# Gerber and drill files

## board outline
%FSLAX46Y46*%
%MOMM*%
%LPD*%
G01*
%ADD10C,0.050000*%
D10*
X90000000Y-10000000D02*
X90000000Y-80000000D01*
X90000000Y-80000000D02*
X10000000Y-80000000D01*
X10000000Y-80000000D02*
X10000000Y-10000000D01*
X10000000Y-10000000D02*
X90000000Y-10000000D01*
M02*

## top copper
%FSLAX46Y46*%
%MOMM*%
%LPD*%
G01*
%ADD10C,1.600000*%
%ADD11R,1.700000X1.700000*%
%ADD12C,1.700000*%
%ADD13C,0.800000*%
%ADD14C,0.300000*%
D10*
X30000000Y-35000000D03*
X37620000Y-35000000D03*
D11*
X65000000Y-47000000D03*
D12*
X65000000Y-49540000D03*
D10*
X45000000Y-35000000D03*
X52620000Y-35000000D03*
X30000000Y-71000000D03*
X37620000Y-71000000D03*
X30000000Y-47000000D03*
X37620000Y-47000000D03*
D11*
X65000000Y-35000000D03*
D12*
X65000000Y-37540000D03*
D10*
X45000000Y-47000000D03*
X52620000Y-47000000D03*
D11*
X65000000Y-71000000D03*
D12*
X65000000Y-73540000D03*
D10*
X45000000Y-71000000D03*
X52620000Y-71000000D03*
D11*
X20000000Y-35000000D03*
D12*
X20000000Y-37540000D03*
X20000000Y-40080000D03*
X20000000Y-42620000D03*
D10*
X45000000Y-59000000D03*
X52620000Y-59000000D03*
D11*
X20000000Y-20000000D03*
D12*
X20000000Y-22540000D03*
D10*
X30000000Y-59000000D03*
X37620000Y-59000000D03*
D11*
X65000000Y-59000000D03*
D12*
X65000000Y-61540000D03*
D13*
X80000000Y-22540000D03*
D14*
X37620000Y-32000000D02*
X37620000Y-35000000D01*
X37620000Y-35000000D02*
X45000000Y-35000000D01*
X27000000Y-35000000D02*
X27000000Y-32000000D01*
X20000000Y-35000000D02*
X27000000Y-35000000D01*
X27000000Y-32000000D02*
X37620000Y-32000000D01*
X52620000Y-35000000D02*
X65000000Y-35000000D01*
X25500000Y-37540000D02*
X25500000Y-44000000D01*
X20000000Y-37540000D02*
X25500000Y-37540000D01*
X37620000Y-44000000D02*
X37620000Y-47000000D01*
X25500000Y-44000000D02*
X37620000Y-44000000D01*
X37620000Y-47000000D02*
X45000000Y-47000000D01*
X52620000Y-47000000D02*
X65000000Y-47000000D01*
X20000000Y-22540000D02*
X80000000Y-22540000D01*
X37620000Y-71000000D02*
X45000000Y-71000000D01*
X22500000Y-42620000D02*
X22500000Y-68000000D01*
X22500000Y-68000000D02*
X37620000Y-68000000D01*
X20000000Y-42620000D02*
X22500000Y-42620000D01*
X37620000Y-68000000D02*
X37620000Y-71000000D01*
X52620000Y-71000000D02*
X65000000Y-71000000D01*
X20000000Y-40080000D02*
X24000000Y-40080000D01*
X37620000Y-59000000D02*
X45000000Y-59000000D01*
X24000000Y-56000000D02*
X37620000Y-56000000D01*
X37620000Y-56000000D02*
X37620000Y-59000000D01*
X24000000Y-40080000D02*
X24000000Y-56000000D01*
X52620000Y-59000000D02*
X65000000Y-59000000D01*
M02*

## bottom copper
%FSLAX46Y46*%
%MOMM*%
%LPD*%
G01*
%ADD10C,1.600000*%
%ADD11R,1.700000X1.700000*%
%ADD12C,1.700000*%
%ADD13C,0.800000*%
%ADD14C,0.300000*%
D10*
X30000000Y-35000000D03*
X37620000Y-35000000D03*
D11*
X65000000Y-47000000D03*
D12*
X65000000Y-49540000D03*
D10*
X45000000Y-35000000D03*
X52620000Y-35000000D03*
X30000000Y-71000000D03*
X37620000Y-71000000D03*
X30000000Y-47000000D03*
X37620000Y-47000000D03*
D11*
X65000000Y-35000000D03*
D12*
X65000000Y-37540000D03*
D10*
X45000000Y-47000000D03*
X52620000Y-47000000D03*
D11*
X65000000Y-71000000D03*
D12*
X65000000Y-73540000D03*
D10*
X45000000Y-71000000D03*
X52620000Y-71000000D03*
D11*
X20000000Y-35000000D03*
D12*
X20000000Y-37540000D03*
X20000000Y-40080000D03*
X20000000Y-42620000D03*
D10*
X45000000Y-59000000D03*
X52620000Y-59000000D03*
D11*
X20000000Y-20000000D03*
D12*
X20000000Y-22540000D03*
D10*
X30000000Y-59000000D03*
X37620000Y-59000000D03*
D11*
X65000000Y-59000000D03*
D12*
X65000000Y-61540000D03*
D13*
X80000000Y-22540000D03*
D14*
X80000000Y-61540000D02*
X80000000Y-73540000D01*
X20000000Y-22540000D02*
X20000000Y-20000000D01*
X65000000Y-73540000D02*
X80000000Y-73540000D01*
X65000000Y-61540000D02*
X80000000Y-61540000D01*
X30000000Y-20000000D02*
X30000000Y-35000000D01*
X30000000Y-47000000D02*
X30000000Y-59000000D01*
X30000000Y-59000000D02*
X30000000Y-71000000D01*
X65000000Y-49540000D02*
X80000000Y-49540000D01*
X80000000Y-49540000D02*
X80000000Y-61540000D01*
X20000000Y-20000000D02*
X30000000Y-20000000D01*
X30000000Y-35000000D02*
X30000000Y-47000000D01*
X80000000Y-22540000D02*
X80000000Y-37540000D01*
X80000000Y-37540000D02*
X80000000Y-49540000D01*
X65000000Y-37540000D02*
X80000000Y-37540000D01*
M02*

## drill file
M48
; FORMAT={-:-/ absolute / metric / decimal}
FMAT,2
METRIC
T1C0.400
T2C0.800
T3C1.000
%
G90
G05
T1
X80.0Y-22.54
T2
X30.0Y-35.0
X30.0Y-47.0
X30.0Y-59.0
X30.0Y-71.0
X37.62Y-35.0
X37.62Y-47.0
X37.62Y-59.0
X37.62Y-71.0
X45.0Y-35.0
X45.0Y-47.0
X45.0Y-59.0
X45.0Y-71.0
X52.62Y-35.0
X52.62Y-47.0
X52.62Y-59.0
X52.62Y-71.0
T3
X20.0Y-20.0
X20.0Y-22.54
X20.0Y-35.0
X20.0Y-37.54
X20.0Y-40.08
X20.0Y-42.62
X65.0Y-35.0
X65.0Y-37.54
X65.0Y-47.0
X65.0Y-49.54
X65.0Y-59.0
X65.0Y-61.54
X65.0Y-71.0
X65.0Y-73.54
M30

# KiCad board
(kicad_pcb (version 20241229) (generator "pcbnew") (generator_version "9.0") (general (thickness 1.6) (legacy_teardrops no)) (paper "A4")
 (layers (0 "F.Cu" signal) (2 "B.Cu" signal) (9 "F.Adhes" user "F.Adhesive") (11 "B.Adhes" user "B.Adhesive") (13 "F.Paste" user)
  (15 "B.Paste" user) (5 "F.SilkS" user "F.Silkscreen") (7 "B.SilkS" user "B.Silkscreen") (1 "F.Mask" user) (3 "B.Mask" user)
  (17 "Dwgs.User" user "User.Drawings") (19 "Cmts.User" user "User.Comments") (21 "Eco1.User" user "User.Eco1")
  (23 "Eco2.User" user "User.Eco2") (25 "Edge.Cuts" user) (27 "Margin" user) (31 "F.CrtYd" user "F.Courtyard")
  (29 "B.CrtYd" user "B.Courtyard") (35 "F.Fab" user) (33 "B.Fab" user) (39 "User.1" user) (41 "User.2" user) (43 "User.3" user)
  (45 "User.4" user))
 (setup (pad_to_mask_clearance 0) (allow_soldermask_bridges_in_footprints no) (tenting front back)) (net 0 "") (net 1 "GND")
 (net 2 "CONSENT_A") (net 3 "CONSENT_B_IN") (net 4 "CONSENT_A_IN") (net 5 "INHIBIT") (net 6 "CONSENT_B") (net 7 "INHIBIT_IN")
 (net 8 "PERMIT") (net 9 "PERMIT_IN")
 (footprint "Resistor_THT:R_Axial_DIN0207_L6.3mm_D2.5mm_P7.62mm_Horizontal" (layer "F.Cu") (at 30 35)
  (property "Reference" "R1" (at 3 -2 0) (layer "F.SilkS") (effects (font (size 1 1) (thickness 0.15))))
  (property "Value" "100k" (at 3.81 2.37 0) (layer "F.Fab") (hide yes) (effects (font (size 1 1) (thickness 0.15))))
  (pad "1" thru_hole circle (at 0 0) (size 1.6 1.6) (drill 0.8) (layers "*.Cu" "*.Mask") (remove_unused_layers no) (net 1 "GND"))
  (pad "2" thru_hole circle (at 7.62 0) (size 1.6 1.6) (drill 0.8) (layers "*.Cu" "*.Mask") (remove_unused_layers no) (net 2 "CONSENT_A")))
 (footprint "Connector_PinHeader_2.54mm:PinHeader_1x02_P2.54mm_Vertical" (layer "F.Cu") (at 65 47)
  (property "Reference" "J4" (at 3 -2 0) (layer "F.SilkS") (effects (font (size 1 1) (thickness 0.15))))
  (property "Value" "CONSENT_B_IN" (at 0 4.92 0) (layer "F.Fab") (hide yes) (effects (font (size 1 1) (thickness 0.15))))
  (pad "1" thru_hole rect (at 0 0) (size 1.7 1.7) (drill 1) (layers "*.Cu" "*.Mask") (remove_unused_layers no) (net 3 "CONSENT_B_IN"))
  (pad "2" thru_hole circle (at 0 2.54) (size 1.7 1.7) (drill 1) (layers "*.Cu" "*.Mask") (remove_unused_layers no) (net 1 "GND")))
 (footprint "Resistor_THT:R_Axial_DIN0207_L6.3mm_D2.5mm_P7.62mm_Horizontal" (layer "F.Cu") (at 45 35)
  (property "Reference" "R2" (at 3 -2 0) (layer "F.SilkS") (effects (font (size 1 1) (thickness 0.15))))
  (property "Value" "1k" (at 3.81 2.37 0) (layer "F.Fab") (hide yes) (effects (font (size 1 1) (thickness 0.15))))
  (pad "1" thru_hole circle (at 0 0) (size 1.6 1.6) (drill 0.8) (layers "*.Cu" "*.Mask") (remove_unused_layers no) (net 2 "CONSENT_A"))
  (pad "2" thru_hole circle (at 7.62 0) (size 1.6 1.6) (drill 0.8) (layers "*.Cu" "*.Mask") (remove_unused_layers no) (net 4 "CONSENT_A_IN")))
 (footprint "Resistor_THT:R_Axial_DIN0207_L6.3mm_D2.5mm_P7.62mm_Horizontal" (layer "F.Cu") (at 30 71)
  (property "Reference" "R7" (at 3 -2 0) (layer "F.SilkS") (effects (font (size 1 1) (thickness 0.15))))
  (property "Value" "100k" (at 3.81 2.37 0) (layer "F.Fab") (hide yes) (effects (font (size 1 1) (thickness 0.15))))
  (pad "1" thru_hole circle (at 0 0) (size 1.6 1.6) (drill 0.8) (layers "*.Cu" "*.Mask") (remove_unused_layers no) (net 1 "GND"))
  (pad "2" thru_hole circle (at 7.62 0) (size 1.6 1.6) (drill 0.8) (layers "*.Cu" "*.Mask") (remove_unused_layers no) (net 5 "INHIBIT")))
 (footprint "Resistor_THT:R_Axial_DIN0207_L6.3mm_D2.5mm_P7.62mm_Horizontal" (layer "F.Cu") (at 30 47)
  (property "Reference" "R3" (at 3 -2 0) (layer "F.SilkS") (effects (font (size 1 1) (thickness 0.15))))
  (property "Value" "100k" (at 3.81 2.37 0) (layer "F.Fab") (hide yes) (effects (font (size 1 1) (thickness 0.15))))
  (pad "1" thru_hole circle (at 0 0) (size 1.6 1.6) (drill 0.8) (layers "*.Cu" "*.Mask") (remove_unused_layers no) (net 1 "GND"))
  (pad "2" thru_hole circle (at 7.62 0) (size 1.6 1.6) (drill 0.8) (layers "*.Cu" "*.Mask") (remove_unused_layers no) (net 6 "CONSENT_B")))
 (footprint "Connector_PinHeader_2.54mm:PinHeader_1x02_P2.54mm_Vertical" (layer "F.Cu") (at 65 35)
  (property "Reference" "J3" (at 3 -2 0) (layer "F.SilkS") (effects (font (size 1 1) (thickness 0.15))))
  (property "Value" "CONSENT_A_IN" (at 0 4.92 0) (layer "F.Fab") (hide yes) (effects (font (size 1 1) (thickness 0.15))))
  (pad "1" thru_hole rect (at 0 0) (size 1.7 1.7) (drill 1) (layers "*.Cu" "*.Mask") (remove_unused_layers no) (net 4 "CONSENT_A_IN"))
  (pad "2" thru_hole circle (at 0 2.54) (size 1.7 1.7) (drill 1) (layers "*.Cu" "*.Mask") (remove_unused_layers no) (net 1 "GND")))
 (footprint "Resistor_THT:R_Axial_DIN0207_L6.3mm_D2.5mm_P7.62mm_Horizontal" (layer "F.Cu") (at 45 47)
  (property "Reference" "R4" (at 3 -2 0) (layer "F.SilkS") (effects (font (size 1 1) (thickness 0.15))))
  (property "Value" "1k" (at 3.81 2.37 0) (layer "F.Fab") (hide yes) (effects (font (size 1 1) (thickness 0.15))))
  (pad "1" thru_hole circle (at 0 0) (size 1.6 1.6) (drill 0.8) (layers "*.Cu" "*.Mask") (remove_unused_layers no) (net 6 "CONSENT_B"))
  (pad "2" thru_hole circle (at 7.62 0) (size 1.6 1.6) (drill 0.8) (layers "*.Cu" "*.Mask") (remove_unused_layers no) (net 3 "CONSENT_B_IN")))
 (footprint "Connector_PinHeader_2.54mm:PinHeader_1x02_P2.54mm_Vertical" (layer "F.Cu") (at 65 71)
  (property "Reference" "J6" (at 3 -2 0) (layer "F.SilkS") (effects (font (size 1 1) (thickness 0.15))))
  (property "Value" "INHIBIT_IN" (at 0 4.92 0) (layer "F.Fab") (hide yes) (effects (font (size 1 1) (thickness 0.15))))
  (pad "1" thru_hole rect (at 0 0) (size 1.7 1.7) (drill 1) (layers "*.Cu" "*.Mask") (remove_unused_layers no) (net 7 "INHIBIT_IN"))
  (pad "2" thru_hole circle (at 0 2.54) (size 1.7 1.7) (drill 1) (layers "*.Cu" "*.Mask") (remove_unused_layers no) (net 1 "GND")))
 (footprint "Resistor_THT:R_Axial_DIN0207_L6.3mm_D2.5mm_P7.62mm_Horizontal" (layer "F.Cu") (at 45 71)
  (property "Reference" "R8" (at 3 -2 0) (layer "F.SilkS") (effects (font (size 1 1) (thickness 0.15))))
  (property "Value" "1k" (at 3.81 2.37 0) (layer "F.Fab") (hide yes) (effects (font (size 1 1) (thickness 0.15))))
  (pad "1" thru_hole circle (at 0 0) (size 1.6 1.6) (drill 0.8) (layers "*.Cu" "*.Mask") (remove_unused_layers no) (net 5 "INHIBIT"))
  (pad "2" thru_hole circle (at 7.62 0) (size 1.6 1.6) (drill 0.8) (layers "*.Cu" "*.Mask") (remove_unused_layers no) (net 7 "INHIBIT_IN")))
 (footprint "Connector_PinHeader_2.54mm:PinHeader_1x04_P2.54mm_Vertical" (layer "F.Cu") (at 20 35)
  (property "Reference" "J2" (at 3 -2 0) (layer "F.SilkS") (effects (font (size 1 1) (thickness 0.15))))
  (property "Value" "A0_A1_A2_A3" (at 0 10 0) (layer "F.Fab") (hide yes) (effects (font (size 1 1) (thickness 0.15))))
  (pad "1" thru_hole rect (at 0 0) (size 1.7 1.7) (drill 1) (layers "*.Cu" "*.Mask") (remove_unused_layers no) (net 2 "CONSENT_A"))
  (pad "2" thru_hole circle (at 0 2.54) (size 1.7 1.7) (drill 1) (layers "*.Cu" "*.Mask") (remove_unused_layers no) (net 6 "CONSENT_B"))
  (pad "3" thru_hole circle (at 0 5.08) (size 1.7 1.7) (drill 1) (layers "*.Cu" "*.Mask") (remove_unused_layers no) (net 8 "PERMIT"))
  (pad "4" thru_hole circle (at 0 7.62) (size 1.7 1.7) (drill 1) (layers "*.Cu" "*.Mask") (remove_unused_layers no) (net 5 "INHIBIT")))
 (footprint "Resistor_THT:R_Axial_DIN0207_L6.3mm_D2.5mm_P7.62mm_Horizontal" (layer "F.Cu") (at 45 59)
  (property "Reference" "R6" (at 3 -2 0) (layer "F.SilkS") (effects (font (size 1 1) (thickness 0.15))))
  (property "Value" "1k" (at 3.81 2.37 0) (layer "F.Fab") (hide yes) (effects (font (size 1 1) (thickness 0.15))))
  (pad "1" thru_hole circle (at 0 0) (size 1.6 1.6) (drill 0.8) (layers "*.Cu" "*.Mask") (remove_unused_layers no) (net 8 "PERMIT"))
  (pad "2" thru_hole circle (at 7.62 0) (size 1.6 1.6) (drill 0.8) (layers "*.Cu" "*.Mask") (remove_unused_layers no) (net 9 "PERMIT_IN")))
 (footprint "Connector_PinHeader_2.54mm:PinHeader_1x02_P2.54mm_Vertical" (layer "F.Cu") (at 20 20)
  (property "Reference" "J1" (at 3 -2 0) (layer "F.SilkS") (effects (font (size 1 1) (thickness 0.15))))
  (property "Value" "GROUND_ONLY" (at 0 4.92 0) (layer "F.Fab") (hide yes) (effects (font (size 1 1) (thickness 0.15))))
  (pad "1" thru_hole rect (at 0 0) (size 1.7 1.7) (drill 1) (layers "*.Cu" "*.Mask") (remove_unused_layers no) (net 1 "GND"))
  (pad "2" thru_hole circle (at 0 2.54) (size 1.7 1.7) (drill 1) (layers "*.Cu" "*.Mask") (remove_unused_layers no) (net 1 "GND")))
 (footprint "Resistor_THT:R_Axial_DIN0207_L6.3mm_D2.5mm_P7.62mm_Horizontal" (layer "F.Cu") (at 30 59)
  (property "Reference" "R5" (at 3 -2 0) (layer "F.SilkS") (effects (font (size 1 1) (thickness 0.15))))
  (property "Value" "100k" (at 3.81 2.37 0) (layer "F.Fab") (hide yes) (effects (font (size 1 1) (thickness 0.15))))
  (pad "1" thru_hole circle (at 0 0) (size 1.6 1.6) (drill 0.8) (layers "*.Cu" "*.Mask") (remove_unused_layers no) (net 1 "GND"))
  (pad "2" thru_hole circle (at 7.62 0) (size 1.6 1.6) (drill 0.8) (layers "*.Cu" "*.Mask") (remove_unused_layers no) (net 8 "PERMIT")))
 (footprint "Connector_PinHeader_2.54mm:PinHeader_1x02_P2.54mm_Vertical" (layer "F.Cu") (at 65 59)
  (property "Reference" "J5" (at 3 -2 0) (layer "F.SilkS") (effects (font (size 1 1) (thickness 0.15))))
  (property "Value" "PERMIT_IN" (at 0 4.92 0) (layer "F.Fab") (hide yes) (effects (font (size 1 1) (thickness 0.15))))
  (pad "1" thru_hole rect (at 0 0) (size 1.7 1.7) (drill 1) (layers "*.Cu" "*.Mask") (remove_unused_layers no) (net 9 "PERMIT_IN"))
  (pad "2" thru_hole circle (at 0 2.54) (size 1.7 1.7) (drill 1) (layers "*.Cu" "*.Mask") (remove_unused_layers no) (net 1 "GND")))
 (gr_line (start 90 10) (end 90 80) (stroke (width 0.05) (type default)) (layer "Edge.Cuts"))
 (gr_line (start 90 80) (end 10 80) (stroke (width 0.05) (type default)) (layer "Edge.Cuts"))
 (gr_line (start 10 80) (end 10 10) (stroke (width 0.05) (type default)) (layer "Edge.Cuts"))
 (gr_line (start 10 10) (end 90 10) (stroke (width 0.05) (type default)) (layer "Edge.Cuts"))
 (segment (start 37.62 32) (end 37.62 35) (width 0.3) (layer "F.Cu") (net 2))
 (segment (start 37.62 35) (end 45 35) (width 0.3) (layer "F.Cu") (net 2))
 (segment (start 27 35) (end 27 32) (width 0.3) (layer "F.Cu") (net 2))
 (segment (start 20 35) (end 27 35) (width 0.3) (layer "F.Cu") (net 2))
 (segment (start 27 32) (end 37.62 32) (width 0.3) (layer "F.Cu") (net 2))
 (segment (start 52.62 35) (end 65 35) (width 0.3) (layer "F.Cu") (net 4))
 (segment (start 25.5 37.54) (end 25.5 44) (width 0.3) (layer "F.Cu") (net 6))
 (segment (start 20 37.54) (end 25.5 37.54) (width 0.3) (layer "F.Cu") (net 6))
 (segment (start 37.62 44) (end 37.62 47) (width 0.3) (layer "F.Cu") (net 6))
 (segment (start 25.5 44) (end 37.62 44) (width 0.3) (layer "F.Cu") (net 6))
 (segment (start 37.62 47) (end 45 47) (width 0.3) (layer "F.Cu") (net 6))
 (segment (start 52.62 47) (end 65 47) (width 0.3) (layer "F.Cu") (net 3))
 (segment (start 20 22.54) (end 80 22.54) (width 0.3) (layer "F.Cu") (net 1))
 (via (at 80 22.54) (size 0.8) (drill 0.4) (layers "F.Cu" "B.Cu") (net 1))
 (segment (start 80 61.54) (end 80 73.54) (width 0.3) (layer "B.Cu") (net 1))
 (segment (start 20 22.54) (end 20 20) (width 0.3) (layer "B.Cu") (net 1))
 (segment (start 65 73.54) (end 80 73.54) (width 0.3) (layer "B.Cu") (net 1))
 (segment (start 65 61.54) (end 80 61.54) (width 0.3) (layer "B.Cu") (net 1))
 (segment (start 30 20) (end 30 35) (width 0.3) (layer "B.Cu") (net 1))
 (segment (start 30 47) (end 30 59) (width 0.3) (layer "B.Cu") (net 1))
 (segment (start 30 59) (end 30 71) (width 0.3) (layer "B.Cu") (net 1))
 (segment (start 65 49.54) (end 80 49.54) (width 0.3) (layer "B.Cu") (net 1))
 (segment (start 80 49.54) (end 80 61.54) (width 0.3) (layer "B.Cu") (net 1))
 (segment (start 20 20) (end 30 20) (width 0.3) (layer "B.Cu") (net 1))
 (segment (start 30 35) (end 30 47) (width 0.3) (layer "B.Cu") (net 1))
 (segment (start 80 22.54) (end 80 37.54) (width 0.3) (layer "B.Cu") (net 1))
 (segment (start 80 37.54) (end 80 49.54) (width 0.3) (layer "B.Cu") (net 1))
 (segment (start 65 37.54) (end 80 37.54) (width 0.3) (layer "B.Cu") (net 1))
 (segment (start 37.62 71) (end 45 71) (width 0.3) (layer "F.Cu") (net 5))
 (segment (start 22.5 42.62) (end 22.5 68) (width 0.3) (layer "F.Cu") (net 5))
 (segment (start 22.5 68) (end 37.62 68) (width 0.3) (layer "F.Cu") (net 5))
 (segment (start 20 42.62) (end 22.5 42.62) (width 0.3) (layer "F.Cu") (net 5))
 (segment (start 37.62 68) (end 37.62 71) (width 0.3) (layer "F.Cu") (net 5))
 (segment (start 52.62 71) (end 65 71) (width 0.3) (layer "F.Cu") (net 7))
 (segment (start 20 40.08) (end 24 40.08) (width 0.3) (layer "F.Cu") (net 8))
 (segment (start 37.62 59) (end 45 59) (width 0.3) (layer "F.Cu") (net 8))
 (segment (start 24 56) (end 37.62 56) (width 0.3) (layer "F.Cu") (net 8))
 (segment (start 37.62 56) (end 37.62 59) (width 0.3) (layer "F.Cu") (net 8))
 (segment (start 24 40.08) (end 24 56) (width 0.3) (layer "F.Cu") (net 8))
 (segment (start 52.62 59) (end 65 59) (width 0.3) (layer "F.Cu") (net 9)))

